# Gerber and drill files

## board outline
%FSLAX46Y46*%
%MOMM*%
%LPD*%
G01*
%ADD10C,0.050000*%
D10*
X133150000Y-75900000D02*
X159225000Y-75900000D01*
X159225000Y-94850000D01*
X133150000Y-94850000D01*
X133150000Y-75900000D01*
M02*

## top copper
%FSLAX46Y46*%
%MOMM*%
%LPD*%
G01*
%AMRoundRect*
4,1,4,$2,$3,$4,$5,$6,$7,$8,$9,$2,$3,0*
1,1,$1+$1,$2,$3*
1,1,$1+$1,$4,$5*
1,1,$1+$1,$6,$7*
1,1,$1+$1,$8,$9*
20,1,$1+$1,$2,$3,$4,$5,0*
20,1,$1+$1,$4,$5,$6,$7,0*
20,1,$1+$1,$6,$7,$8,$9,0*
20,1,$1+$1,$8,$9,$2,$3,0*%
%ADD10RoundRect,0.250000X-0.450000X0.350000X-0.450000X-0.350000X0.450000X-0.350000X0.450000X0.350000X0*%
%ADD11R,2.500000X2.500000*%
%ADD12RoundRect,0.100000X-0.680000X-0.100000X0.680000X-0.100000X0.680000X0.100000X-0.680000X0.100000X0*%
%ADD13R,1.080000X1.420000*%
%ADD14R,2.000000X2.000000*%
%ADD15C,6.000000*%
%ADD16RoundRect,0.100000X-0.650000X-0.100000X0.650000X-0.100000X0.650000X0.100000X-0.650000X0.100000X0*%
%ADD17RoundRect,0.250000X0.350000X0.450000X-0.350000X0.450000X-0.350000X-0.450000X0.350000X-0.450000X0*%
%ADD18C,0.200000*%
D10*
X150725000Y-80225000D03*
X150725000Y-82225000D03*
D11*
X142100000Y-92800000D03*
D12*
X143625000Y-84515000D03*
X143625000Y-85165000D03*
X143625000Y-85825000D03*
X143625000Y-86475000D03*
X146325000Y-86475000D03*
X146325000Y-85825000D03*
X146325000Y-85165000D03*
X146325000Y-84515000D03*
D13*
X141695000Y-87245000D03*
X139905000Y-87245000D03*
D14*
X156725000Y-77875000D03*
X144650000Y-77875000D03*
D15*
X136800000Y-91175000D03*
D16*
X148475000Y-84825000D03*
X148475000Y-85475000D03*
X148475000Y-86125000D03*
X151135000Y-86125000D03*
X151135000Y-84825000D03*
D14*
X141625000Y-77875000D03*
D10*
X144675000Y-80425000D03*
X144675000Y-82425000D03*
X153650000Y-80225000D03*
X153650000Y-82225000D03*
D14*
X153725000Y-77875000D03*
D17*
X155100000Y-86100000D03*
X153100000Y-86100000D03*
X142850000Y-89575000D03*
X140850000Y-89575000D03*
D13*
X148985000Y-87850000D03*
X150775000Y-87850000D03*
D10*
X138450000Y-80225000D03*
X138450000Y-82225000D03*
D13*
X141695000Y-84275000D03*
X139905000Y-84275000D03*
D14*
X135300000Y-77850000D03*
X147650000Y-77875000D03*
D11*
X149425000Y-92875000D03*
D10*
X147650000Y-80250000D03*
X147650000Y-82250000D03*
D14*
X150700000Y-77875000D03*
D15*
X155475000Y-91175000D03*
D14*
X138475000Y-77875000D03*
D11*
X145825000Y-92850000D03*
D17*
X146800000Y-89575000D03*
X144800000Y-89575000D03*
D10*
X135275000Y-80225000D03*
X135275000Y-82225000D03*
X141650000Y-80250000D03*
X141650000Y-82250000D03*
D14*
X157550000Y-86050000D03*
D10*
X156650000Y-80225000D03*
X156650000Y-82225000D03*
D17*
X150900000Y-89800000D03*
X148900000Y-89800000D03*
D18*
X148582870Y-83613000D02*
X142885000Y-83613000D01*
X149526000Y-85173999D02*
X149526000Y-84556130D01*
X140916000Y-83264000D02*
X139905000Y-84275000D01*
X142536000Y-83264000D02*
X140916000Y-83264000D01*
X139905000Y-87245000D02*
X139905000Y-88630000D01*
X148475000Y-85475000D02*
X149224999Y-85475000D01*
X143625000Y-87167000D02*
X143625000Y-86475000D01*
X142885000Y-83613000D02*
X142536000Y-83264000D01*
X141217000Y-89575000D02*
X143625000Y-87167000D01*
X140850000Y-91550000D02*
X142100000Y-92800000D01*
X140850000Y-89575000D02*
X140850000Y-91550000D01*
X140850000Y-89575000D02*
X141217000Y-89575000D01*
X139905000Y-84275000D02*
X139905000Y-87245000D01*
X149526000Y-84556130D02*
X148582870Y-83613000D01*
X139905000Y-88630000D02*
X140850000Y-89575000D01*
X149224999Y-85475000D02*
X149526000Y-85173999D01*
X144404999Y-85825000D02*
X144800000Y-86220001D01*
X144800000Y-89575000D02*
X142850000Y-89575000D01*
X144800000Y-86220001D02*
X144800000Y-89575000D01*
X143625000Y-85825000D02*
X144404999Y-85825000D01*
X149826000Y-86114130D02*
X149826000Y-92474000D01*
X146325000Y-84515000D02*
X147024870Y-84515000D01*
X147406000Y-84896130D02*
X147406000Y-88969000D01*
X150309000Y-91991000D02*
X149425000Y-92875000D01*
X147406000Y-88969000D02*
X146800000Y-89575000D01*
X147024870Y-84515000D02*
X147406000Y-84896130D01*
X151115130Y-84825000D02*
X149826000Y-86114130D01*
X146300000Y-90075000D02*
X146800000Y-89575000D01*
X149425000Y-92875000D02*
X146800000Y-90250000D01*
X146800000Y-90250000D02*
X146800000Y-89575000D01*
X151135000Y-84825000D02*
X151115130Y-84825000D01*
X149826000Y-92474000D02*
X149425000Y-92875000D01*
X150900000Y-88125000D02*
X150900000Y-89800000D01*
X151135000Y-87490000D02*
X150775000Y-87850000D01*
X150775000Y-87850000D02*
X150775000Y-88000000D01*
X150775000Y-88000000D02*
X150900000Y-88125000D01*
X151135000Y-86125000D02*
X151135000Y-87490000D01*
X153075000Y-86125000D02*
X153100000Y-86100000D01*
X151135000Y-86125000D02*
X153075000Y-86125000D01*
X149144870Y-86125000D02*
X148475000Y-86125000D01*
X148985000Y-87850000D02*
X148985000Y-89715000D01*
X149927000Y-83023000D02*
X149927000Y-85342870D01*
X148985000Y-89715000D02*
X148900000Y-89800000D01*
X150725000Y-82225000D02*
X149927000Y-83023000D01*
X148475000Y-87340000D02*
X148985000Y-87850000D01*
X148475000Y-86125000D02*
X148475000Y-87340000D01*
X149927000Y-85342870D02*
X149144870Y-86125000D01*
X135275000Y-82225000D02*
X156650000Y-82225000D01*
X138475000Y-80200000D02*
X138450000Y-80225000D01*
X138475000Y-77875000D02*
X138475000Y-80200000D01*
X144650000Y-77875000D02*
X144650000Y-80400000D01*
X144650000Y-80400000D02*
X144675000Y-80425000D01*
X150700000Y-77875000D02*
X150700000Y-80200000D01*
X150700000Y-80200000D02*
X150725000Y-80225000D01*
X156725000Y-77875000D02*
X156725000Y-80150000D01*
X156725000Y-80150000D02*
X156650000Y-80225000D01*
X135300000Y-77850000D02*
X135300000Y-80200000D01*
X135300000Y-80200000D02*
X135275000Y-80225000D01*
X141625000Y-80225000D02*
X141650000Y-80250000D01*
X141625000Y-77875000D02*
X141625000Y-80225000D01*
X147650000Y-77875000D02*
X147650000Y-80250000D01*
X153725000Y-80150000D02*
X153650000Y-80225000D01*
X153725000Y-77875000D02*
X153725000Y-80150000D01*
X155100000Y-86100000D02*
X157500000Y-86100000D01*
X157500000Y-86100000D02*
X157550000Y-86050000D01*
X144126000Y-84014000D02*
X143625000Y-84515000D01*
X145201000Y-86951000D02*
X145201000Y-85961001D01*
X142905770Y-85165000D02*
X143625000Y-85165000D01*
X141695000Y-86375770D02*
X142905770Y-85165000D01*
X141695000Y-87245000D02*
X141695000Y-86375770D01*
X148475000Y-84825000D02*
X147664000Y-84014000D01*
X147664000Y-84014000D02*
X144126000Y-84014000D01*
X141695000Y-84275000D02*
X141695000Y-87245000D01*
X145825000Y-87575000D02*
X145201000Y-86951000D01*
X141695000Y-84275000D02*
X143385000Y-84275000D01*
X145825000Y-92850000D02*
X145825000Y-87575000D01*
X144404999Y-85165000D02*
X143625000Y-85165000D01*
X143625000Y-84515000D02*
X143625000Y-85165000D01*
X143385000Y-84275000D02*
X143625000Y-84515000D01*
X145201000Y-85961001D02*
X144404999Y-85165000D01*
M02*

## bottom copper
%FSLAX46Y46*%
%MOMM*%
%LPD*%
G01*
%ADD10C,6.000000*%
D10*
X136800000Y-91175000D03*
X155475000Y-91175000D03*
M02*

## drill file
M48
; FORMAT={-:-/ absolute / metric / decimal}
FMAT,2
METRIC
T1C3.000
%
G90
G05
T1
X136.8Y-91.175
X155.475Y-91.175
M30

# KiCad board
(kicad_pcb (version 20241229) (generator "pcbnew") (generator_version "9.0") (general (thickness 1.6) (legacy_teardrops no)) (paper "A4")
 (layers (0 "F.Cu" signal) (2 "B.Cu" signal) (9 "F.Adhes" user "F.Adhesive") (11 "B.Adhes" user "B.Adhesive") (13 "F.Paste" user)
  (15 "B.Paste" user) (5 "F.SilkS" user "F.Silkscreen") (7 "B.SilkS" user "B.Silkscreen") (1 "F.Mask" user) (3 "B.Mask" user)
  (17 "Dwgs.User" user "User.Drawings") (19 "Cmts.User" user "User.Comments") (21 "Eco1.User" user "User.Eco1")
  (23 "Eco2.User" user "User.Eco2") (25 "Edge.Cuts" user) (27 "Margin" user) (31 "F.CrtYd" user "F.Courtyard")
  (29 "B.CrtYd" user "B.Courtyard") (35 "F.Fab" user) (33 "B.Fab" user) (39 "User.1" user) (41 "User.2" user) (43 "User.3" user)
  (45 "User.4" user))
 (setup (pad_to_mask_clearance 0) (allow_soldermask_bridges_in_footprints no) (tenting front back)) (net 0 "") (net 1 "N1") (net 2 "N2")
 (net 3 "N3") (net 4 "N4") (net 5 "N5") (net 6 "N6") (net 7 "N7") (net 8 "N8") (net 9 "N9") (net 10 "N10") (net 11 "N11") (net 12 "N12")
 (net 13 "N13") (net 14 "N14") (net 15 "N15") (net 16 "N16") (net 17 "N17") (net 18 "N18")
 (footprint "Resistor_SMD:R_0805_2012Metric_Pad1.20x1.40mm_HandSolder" (layer "F.Cu") (at 150.725 81.225 -90)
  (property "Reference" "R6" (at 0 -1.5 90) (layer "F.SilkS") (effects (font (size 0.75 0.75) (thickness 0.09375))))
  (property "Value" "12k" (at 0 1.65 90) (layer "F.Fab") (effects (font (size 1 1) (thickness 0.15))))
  (pad "1" smd roundrect (at -1 0 270) (size 1.2 1.4) (layers "F.Cu" "F.Mask" "F.Paste") (roundrect_rratio 0.208333) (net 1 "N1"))
  (pad "2" smd roundrect (at 1 0 270) (size 1.2 1.4) (layers "F.Cu" "F.Mask" "F.Paste") (roundrect_rratio 0.208333) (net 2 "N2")))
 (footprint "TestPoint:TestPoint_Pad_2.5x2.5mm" (layer "F.Cu") (at 142.1 92.8)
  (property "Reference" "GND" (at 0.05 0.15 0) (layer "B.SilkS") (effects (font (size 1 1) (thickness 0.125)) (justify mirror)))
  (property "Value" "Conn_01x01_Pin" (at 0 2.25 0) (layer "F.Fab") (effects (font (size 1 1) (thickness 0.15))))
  (pad "1" smd rect (at 0 0) (size 2.5 2.5) (layers "F.Cu" "F.Mask") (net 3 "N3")))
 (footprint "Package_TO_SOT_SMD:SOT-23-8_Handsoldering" (layer "F.Cu") (at 144.975 85.495)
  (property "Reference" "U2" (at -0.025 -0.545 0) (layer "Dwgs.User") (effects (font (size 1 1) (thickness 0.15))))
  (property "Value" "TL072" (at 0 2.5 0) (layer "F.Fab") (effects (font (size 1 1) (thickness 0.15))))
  (pad "1" smd roundrect (at -1.35 -0.98) (size 1.56 0.4) (layers "F.Cu" "F.Mask" "F.Paste") (roundrect_rratio 0.25) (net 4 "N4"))
  (pad "2" smd roundrect (at -1.35 -0.33) (size 1.56 0.4) (layers "F.Cu" "F.Mask" "F.Paste") (roundrect_rratio 0.25) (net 4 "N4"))
  (pad "3" smd roundrect (at -1.35 0.33) (size 1.56 0.4) (layers "F.Cu" "F.Mask" "F.Paste") (roundrect_rratio 0.25) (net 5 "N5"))
  (pad "4" smd roundrect (at -1.35 0.98) (size 1.56 0.4) (layers "F.Cu" "F.Mask" "F.Paste") (roundrect_rratio 0.25) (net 3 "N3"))
  (pad "5" smd roundrect (at 1.35 0.98) (size 1.56 0.4) (layers "F.Cu" "F.Mask" "F.Paste") (roundrect_rratio 0.25) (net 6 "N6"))
  (pad "6" smd roundrect (at 1.35 0.33) (size 1.56 0.4) (layers "F.Cu" "F.Mask" "F.Paste") (roundrect_rratio 0.25) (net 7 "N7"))
  (pad "7" smd roundrect (at 1.35 -0.33) (size 1.56 0.4) (layers "F.Cu" "F.Mask" "F.Paste") (roundrect_rratio 0.25) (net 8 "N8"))
  (pad "8" smd roundrect (at 1.35 -0.98) (size 1.56 0.4) (layers "F.Cu" "F.Mask" "F.Paste") (roundrect_rratio 0.25) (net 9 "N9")))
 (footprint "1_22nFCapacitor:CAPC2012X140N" (layer "F.Cu") (at 140.8 87.245 180)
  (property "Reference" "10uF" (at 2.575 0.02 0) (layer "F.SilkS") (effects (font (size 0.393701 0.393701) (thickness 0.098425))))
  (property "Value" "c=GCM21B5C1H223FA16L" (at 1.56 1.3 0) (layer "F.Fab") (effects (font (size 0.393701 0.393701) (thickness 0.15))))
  (pad "1" smd rect (at -0.895 0 180) (size 1.08 1.42) (layers "F.Cu" "F.Mask" "F.Paste") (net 4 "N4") (solder_mask_margin 0.102))
  (pad "2" smd rect (at 0.895 0 180) (size 1.08 1.42) (layers "F.Cu" "F.Mask" "F.Paste") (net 3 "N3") (solder_mask_margin 0.102)))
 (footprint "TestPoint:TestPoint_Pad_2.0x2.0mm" (layer "F.Cu") (at 156.725 77.875)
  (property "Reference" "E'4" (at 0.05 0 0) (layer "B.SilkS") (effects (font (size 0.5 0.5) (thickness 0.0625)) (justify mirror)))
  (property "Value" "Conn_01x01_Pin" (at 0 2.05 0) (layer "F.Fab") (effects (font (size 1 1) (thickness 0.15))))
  (pad "1" smd rect (at 0 0) (size 2 2) (layers "F.Cu" "F.Mask") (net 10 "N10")))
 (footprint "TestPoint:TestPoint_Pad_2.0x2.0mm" (layer "F.Cu") (at 144.65 77.875)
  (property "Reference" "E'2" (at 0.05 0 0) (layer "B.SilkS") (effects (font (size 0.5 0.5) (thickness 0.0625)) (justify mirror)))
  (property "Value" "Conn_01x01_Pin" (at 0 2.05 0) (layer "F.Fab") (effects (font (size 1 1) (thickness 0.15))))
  (pad "1" smd rect (at 0 0) (size 2 2) (layers "F.Cu" "F.Mask") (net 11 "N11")))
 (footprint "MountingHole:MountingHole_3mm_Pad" (layer "F.Cu") (at 136.8 91.175)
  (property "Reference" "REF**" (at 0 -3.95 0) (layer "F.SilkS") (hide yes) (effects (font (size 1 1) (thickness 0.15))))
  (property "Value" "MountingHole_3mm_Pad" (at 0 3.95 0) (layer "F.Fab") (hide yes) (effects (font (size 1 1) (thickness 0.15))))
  (pad "1" thru_hole circle (at 0 0) (size 6 6) (drill 3) (layers "*.Cu" "*.Mask") (remove_unused_layers no) (zone_connect 2)))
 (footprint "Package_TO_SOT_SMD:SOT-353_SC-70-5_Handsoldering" (layer "F.Cu") (at 149.805 85.475)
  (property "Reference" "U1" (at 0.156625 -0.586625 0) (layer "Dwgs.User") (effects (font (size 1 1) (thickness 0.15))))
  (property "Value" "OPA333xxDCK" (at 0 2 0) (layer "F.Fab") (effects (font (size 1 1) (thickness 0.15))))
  (pad "1" smd roundrect (at -1.33 -0.65) (size 1.5 0.4) (layers "F.Cu" "F.Mask" "F.Paste") (roundrect_rratio 0.25) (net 4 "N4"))
  (pad "2" smd roundrect (at -1.33 0) (size 1.5 0.4) (layers "F.Cu" "F.Mask" "F.Paste") (roundrect_rratio 0.25) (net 3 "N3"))
  (pad "3" smd roundrect (at -1.33 0.65) (size 1.5 0.4) (layers "F.Cu" "F.Mask" "F.Paste") (roundrect_rratio 0.25) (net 2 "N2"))
  (pad "4" smd roundrect (at 1.33 0.65) (size 1.5 0.4) (layers "F.Cu" "F.Mask" "F.Paste") (roundrect_rratio 0.25) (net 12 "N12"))
  (pad "5" smd roundrect (at 1.33 -0.65) (size 1.5 0.4) (layers "F.Cu" "F.Mask" "F.Paste") (roundrect_rratio 0.25) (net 9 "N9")))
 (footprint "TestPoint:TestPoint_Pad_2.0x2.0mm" (layer "F.Cu") (at 141.625 77.875)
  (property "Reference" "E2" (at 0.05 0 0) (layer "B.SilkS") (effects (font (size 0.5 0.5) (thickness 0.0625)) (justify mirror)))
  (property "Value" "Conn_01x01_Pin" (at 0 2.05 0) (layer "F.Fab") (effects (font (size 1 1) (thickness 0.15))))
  (pad "1" smd rect (at 0 0) (size 2 2) (layers "F.Cu" "F.Mask") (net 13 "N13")))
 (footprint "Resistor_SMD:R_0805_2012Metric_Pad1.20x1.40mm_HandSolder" (layer "F.Cu") (at 144.675 81.425 -90)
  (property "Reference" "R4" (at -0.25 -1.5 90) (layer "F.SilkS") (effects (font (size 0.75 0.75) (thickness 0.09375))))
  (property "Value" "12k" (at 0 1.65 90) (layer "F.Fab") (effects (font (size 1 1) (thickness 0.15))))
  (pad "1" smd roundrect (at -1 0 270) (size 1.2 1.4) (layers "F.Cu" "F.Mask" "F.Paste") (roundrect_rratio 0.208333) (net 11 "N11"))
  (pad "2" smd roundrect (at 1 0 270) (size 1.2 1.4) (layers "F.Cu" "F.Mask" "F.Paste") (roundrect_rratio 0.208333) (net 2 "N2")))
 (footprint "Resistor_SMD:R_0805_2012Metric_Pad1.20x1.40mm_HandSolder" (layer "F.Cu") (at 153.65 81.225 -90)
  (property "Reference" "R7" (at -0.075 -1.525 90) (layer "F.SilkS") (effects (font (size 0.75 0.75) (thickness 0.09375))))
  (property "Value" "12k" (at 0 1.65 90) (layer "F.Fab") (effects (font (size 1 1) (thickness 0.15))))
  (pad "1" smd roundrect (at -1 0 270) (size 1.2 1.4) (layers "F.Cu" "F.Mask" "F.Paste") (roundrect_rratio 0.208333) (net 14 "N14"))
  (pad "2" smd roundrect (at 1 0 270) (size 1.2 1.4) (layers "F.Cu" "F.Mask" "F.Paste") (roundrect_rratio 0.208333) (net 2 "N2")))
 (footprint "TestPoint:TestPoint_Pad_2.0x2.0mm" (layer "F.Cu") (at 153.725 77.875)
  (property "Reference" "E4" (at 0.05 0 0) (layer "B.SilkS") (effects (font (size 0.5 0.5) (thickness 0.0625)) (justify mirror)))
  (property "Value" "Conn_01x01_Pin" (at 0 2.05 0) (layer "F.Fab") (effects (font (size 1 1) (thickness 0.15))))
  (pad "1" smd rect (at 0 0) (size 2 2) (layers "F.Cu" "F.Mask") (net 14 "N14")))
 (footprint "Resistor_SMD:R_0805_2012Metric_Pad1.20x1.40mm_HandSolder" (layer "F.Cu") (at 154.1 86.1 180)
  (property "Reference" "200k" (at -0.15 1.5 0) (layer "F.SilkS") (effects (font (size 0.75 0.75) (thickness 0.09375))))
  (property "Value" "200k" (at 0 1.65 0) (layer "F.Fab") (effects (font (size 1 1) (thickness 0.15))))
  (pad "1" smd roundrect (at -1 0 180) (size 1.2 1.4) (layers "F.Cu" "F.Mask" "F.Paste") (roundrect_rratio 0.208333) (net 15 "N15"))
  (pad "2" smd roundrect (at 1 0 180) (size 1.2 1.4) (layers "F.Cu" "F.Mask" "F.Paste") (roundrect_rratio 0.208333) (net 12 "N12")))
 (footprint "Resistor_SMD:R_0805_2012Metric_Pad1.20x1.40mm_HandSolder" (layer "F.Cu") (at 141.85 89.575 180)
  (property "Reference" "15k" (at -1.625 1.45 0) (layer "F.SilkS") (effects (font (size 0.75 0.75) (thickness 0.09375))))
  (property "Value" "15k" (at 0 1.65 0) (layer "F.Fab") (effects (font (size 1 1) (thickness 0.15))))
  (pad "1" smd roundrect (at -1 0 180) (size 1.2 1.4) (layers "F.Cu" "F.Mask" "F.Paste") (roundrect_rratio 0.208333) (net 5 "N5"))
  (pad "2" smd roundrect (at 1 0 180) (size 1.2 1.4) (layers "F.Cu" "F.Mask" "F.Paste") (roundrect_rratio 0.208333) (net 3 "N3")))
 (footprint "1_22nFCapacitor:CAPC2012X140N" (layer "F.Cu") (at 149.88 87.85)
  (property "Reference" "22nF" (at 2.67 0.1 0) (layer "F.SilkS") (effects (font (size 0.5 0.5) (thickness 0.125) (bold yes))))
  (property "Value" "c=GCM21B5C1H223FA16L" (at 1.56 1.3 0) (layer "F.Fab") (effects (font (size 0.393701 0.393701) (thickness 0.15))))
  (pad "1" smd rect (at -0.895 0) (size 1.08 1.42) (layers "F.Cu" "F.Mask" "F.Paste") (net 2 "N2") (solder_mask_margin 0.102))
  (pad "2" smd rect (at 0.895 0) (size 1.08 1.42) (layers "F.Cu" "F.Mask" "F.Paste") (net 12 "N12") (solder_mask_margin 0.102)))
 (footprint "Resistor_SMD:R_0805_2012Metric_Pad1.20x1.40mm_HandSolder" (layer "F.Cu") (at 138.45 81.225 -90)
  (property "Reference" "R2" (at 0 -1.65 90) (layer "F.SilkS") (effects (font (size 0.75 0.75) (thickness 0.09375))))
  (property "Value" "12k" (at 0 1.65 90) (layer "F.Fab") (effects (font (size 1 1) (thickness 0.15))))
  (pad "1" smd roundrect (at -1 0 270) (size 1.2 1.4) (layers "F.Cu" "F.Mask" "F.Paste") (roundrect_rratio 0.208333) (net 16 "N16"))
  (pad "2" smd roundrect (at 1 0 270) (size 1.2 1.4) (layers "F.Cu" "F.Mask" "F.Paste") (roundrect_rratio 0.208333) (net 2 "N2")))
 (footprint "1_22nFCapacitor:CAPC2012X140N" (layer "F.Cu") (at 140.8 84.275 180)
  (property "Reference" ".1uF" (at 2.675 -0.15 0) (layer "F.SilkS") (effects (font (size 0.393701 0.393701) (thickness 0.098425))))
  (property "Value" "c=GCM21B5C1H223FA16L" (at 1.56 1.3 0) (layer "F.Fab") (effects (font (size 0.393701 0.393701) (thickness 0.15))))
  (pad "1" smd rect (at -0.895 0 180) (size 1.08 1.42) (layers "F.Cu" "F.Mask" "F.Paste") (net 4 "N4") (solder_mask_margin 0.102))
  (pad "2" smd rect (at 0.895 0 180) (size 1.08 1.42) (layers "F.Cu" "F.Mask" "F.Paste") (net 3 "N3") (solder_mask_margin 0.102)))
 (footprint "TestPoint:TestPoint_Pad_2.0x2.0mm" (layer "F.Cu") (at 135.3 77.85)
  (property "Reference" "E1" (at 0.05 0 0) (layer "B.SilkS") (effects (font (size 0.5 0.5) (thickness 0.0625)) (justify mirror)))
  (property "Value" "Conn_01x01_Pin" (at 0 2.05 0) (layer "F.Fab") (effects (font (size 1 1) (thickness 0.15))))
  (pad "1" smd rect (at 0 0) (size 2 2) (layers "F.Cu" "F.Mask") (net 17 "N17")))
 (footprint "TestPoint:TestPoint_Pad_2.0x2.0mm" (layer "F.Cu") (at 147.65 77.875)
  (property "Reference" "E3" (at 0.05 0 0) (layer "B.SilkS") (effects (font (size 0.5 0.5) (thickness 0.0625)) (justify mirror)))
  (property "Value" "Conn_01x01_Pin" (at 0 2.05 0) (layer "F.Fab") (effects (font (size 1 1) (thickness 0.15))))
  (pad "1" smd rect (at 0 0) (size 2 2) (layers "F.Cu" "F.Mask") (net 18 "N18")))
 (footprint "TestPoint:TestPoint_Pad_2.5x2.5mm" (layer "F.Cu") (at 149.425 92.875)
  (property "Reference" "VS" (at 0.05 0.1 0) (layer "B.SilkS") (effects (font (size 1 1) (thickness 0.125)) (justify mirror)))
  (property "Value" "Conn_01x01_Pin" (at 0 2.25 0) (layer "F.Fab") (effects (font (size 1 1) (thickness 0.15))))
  (pad "1" smd rect (at 0 0) (size 2.5 2.5) (layers "F.Cu" "F.Mask") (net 9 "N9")))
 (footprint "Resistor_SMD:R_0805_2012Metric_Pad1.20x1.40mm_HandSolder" (layer "F.Cu") (at 147.65 81.25 -90)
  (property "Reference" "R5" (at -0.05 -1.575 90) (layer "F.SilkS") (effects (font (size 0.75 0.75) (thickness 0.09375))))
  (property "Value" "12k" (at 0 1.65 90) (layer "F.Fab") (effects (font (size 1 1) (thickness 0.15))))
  (pad "1" smd roundrect (at -1 0 270) (size 1.2 1.4) (layers "F.Cu" "F.Mask" "F.Paste") (roundrect_rratio 0.208333) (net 18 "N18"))
  (pad "2" smd roundrect (at 1 0 270) (size 1.2 1.4) (layers "F.Cu" "F.Mask" "F.Paste") (roundrect_rratio 0.208333) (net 2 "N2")))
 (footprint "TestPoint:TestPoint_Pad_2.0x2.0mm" (layer "F.Cu") (at 150.7 77.875)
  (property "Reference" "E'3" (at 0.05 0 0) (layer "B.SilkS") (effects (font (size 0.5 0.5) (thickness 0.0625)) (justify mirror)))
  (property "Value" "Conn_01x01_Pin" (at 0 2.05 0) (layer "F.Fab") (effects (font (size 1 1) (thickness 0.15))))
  (pad "1" smd rect (at 0 0) (size 2 2) (layers "F.Cu" "F.Mask") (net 1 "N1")))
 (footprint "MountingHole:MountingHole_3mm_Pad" (layer "F.Cu") (at 155.475 91.175)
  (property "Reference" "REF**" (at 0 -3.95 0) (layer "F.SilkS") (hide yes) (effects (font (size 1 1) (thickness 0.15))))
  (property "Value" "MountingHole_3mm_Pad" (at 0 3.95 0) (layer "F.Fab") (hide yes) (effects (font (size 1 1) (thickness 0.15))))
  (pad "1" thru_hole circle (at 0 0) (size 6 6) (drill 3) (layers "*.Cu" "*.Mask") (remove_unused_layers no) (zone_connect 2)))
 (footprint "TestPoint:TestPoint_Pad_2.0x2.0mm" (layer "F.Cu") (at 138.475 77.875)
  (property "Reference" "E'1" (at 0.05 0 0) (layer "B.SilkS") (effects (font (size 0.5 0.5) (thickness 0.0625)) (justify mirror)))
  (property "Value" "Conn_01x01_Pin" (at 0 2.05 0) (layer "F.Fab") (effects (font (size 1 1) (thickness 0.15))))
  (pad "1" smd rect (at 0 0) (size 2 2) (layers "F.Cu" "F.Mask") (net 16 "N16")))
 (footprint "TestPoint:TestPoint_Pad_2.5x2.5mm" (layer "F.Cu") (at 145.825 92.85)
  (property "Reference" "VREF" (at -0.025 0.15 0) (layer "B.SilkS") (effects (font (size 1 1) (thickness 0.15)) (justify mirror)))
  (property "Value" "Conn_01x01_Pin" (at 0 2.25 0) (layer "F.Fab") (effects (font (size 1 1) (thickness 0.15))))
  (pad "1" smd rect (at 0 0) (size 2.5 2.5) (layers "F.Cu" "F.Mask") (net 4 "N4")))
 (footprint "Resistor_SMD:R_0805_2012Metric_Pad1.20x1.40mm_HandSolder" (layer "F.Cu") (at 145.8 89.575 180)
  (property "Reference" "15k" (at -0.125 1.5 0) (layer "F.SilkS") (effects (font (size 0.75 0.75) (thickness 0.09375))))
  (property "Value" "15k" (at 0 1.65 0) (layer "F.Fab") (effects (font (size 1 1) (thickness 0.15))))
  (pad "1" smd roundrect (at -1 0 180) (size 1.2 1.4) (layers "F.Cu" "F.Mask" "F.Paste") (roundrect_rratio 0.208333) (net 9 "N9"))
  (pad "2" smd roundrect (at 1 0 180) (size 1.2 1.4) (layers "F.Cu" "F.Mask" "F.Paste") (roundrect_rratio 0.208333) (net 5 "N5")))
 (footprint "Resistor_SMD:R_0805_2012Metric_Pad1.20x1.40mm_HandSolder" (layer "F.Cu") (at 135.275 81.225 -90)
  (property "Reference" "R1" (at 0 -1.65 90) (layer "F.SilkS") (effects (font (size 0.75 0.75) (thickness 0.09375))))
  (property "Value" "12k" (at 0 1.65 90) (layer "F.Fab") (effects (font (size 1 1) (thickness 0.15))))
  (pad "1" smd roundrect (at -1 0 270) (size 1.2 1.4) (layers "F.Cu" "F.Mask" "F.Paste") (roundrect_rratio 0.208333) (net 17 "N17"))
  (pad "2" smd roundrect (at 1 0 270) (size 1.2 1.4) (layers "F.Cu" "F.Mask" "F.Paste") (roundrect_rratio 0.208333) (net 2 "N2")))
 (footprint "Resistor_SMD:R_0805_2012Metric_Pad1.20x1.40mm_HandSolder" (layer "F.Cu") (at 141.65 81.25 -90)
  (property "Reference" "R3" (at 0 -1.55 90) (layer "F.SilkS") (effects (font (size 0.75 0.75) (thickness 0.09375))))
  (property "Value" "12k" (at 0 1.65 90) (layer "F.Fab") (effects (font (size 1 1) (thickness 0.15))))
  (pad "1" smd roundrect (at -1 0 270) (size 1.2 1.4) (layers "F.Cu" "F.Mask" "F.Paste") (roundrect_rratio 0.208333) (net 13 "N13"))
  (pad "2" smd roundrect (at 1 0 270) (size 1.2 1.4) (layers "F.Cu" "F.Mask" "F.Paste") (roundrect_rratio 0.208333) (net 2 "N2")))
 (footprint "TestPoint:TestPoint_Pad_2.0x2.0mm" (layer "F.Cu") (at 157.55 86.05)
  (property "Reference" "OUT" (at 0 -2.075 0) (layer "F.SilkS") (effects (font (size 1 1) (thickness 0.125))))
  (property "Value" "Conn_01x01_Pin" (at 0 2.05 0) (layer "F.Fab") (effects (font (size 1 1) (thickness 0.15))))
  (pad "1" smd rect (at 0 0) (size 2 2) (layers "F.Cu" "F.Mask") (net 15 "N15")))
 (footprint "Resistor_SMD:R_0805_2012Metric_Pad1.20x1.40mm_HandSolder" (layer "F.Cu") (at 156.65 81.225 -90)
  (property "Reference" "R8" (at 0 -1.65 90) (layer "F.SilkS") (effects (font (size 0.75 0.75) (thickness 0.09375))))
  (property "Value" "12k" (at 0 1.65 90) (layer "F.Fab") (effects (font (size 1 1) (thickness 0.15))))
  (pad "1" smd roundrect (at -1 0 270) (size 1.2 1.4) (layers "F.Cu" "F.Mask" "F.Paste") (roundrect_rratio 0.208333) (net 10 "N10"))
  (pad "2" smd roundrect (at 1 0 270) (size 1.2 1.4) (layers "F.Cu" "F.Mask" "F.Paste") (roundrect_rratio 0.208333) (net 2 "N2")))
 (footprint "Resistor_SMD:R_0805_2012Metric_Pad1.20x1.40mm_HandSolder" (layer "F.Cu") (at 149.9 89.8 180)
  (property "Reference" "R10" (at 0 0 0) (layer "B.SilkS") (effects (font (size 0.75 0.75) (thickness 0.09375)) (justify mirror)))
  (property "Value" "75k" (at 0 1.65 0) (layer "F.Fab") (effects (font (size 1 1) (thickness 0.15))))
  (pad "1" smd roundrect (at -1 0 180) (size 1.2 1.4) (layers "F.Cu" "F.Mask" "F.Paste") (roundrect_rratio 0.208333) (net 12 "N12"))
  (pad "2" smd roundrect (at 1 0 180) (size 1.2 1.4) (layers "F.Cu" "F.Mask" "F.Paste") (roundrect_rratio 0.208333) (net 2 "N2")))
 (gr_rect (start 133.15 75.9) (end 159.225 94.85) (stroke (width 0.05) (type solid)) (fill no) (layer "Edge.Cuts"))
 (segment (start 148.58287 83.613) (end 142.885 83.613) (width 0.2) (layer "F.Cu") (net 3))
 (segment (start 149.526 85.173999) (end 149.526 84.55613) (width 0.2) (layer "F.Cu") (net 3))
 (segment (start 140.916 83.264) (end 139.905 84.275) (width 0.2) (layer "F.Cu") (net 3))
 (segment (start 142.536 83.264) (end 140.916 83.264) (width 0.2) (layer "F.Cu") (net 3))
 (segment (start 139.905 87.245) (end 139.905 88.63) (width 0.2) (layer "F.Cu") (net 3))
 (segment (start 148.475 85.475) (end 149.224999 85.475) (width 0.2) (layer "F.Cu") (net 3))
 (segment (start 143.625 87.167) (end 143.625 86.475) (width 0.2) (layer "F.Cu") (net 3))
 (segment (start 142.885 83.613) (end 142.536 83.264) (width 0.2) (layer "F.Cu") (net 3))
 (segment (start 141.217 89.575) (end 143.625 87.167) (width 0.2) (layer "F.Cu") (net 3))
 (segment (start 140.85 91.55) (end 142.1 92.8) (width 0.2) (layer "F.Cu") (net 3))
 (segment (start 140.85 89.575) (end 140.85 91.55) (width 0.2) (layer "F.Cu") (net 3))
 (segment (start 140.85 89.575) (end 141.217 89.575) (width 0.2) (layer "F.Cu") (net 3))
 (segment (start 139.905 84.275) (end 139.905 87.245) (width 0.2) (layer "F.Cu") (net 3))
 (segment (start 149.526 84.55613) (end 148.58287 83.613) (width 0.2) (layer "F.Cu") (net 3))
 (segment (start 139.905 88.63) (end 140.85 89.575) (width 0.2) (layer "F.Cu") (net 3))
 (segment (start 149.224999 85.475) (end 149.526 85.173999) (width 0.2) (layer "F.Cu") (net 3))
 (segment (start 144.404999 85.825) (end 144.8 86.220001) (width 0.2) (layer "F.Cu") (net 5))
 (segment (start 144.8 89.575) (end 142.85 89.575) (width 0.2) (layer "F.Cu") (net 5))
 (segment (start 144.8 86.220001) (end 144.8 89.575) (width 0.2) (layer "F.Cu") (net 5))
 (segment (start 143.625 85.825) (end 144.404999 85.825) (width 0.2) (layer "F.Cu") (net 5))
 (segment (start 149.826 86.11413) (end 149.826 92.474) (width 0.2) (layer "F.Cu") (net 9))
 (segment (start 146.325 84.515) (end 147.02487 84.515) (width 0.2) (layer "F.Cu") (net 9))
 (segment (start 147.406 84.89613) (end 147.406 88.969) (width 0.2) (layer "F.Cu") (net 9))
 (segment (start 150.309 91.991) (end 149.425 92.875) (width 0.2) (layer "F.Cu") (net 9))
 (segment (start 147.406 88.969) (end 146.8 89.575) (width 0.2) (layer "F.Cu") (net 9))
 (segment (start 147.02487 84.515) (end 147.406 84.89613) (width 0.2) (layer "F.Cu") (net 9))
 (segment (start 151.11513 84.825) (end 149.826 86.11413) (width 0.2) (layer "F.Cu") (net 9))
 (segment (start 146.3 90.075) (end 146.8 89.575) (width 0.2) (layer "F.Cu") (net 9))
 (segment (start 149.425 92.875) (end 146.8 90.25) (width 0.2) (layer "F.Cu") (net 9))
 (segment (start 146.8 90.25) (end 146.8 89.575) (width 0.2) (layer "F.Cu") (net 9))
 (segment (start 151.135 84.825) (end 151.11513 84.825) (width 0.2) (layer "F.Cu") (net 9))
 (segment (start 149.826 92.474) (end 149.425 92.875) (width 0.2) (layer "F.Cu") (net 9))
 (segment (start 150.9 88.125) (end 150.9 89.8) (width 0.2) (layer "F.Cu") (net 12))
 (segment (start 151.135 87.49) (end 150.775 87.85) (width 0.2) (layer "F.Cu") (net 12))
 (segment (start 150.775 87.85) (end 150.775 88) (width 0.2) (layer "F.Cu") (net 12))
 (segment (start 150.775 88) (end 150.9 88.125) (width 0.2) (layer "F.Cu") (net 12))
 (segment (start 151.135 86.125) (end 151.135 87.49) (width 0.2) (layer "F.Cu") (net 12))
 (segment (start 153.075 86.125) (end 153.1 86.1) (width 0.2) (layer "F.Cu") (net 12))
 (segment (start 151.135 86.125) (end 153.075 86.125) (width 0.2) (layer "F.Cu") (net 12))
 (segment (start 149.14487 86.125) (end 148.475 86.125) (width 0.2) (layer "F.Cu") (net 2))
 (segment (start 148.985 87.85) (end 148.985 89.715) (width 0.2) (layer "F.Cu") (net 2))
 (segment (start 149.927 83.023) (end 149.927 85.34287) (width 0.2) (layer "F.Cu") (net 2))
 (segment (start 148.985 89.715) (end 148.9 89.8) (width 0.2) (layer "F.Cu") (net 2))
 (segment (start 150.725 82.225) (end 149.927 83.023) (width 0.2) (layer "F.Cu") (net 2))
 (segment (start 148.475 87.34) (end 148.985 87.85) (width 0.2) (layer "F.Cu") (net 2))
 (segment (start 148.475 86.125) (end 148.475 87.34) (width 0.2) (layer "F.Cu") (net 2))
 (segment (start 149.927 85.34287) (end 149.14487 86.125) (width 0.2) (layer "F.Cu") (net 2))
 (segment (start 135.275 82.225) (end 156.65 82.225) (width 0.2) (layer "F.Cu") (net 2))
 (segment (start 138.475 80.2) (end 138.45 80.225) (width 0.2) (layer "F.Cu") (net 16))
 (segment (start 138.475 77.875) (end 138.475 80.2) (width 0.2) (layer "F.Cu") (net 16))
 (segment (start 144.65 77.875) (end 144.65 80.4) (width 0.2) (layer "F.Cu") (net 11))
 (segment (start 144.65 80.4) (end 144.675 80.425) (width 0.2) (layer "F.Cu") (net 11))
 (segment (start 150.7 77.875) (end 150.7 80.2) (width 0.2) (layer "F.Cu") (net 1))
 (segment (start 150.7 80.2) (end 150.725 80.225) (width 0.2) (layer "F.Cu") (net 1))
 (segment (start 156.725 77.875) (end 156.725 80.15) (width 0.2) (layer "F.Cu") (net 10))
 (segment (start 156.725 80.15) (end 156.65 80.225) (width 0.2) (layer "F.Cu") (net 10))
 (segment (start 135.3 77.85) (end 135.3 80.2) (width 0.2) (layer "F.Cu") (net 17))
 (segment (start 135.3 80.2) (end 135.275 80.225) (width 0.2) (layer "F.Cu") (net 17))
 (segment (start 141.625 80.225) (end 141.65 80.25) (width 0.2) (layer "F.Cu") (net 13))
 (segment (start 141.625 77.875) (end 141.625 80.225) (width 0.2) (layer "F.Cu") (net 13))
 (segment (start 147.65 77.875) (end 147.65 80.25) (width 0.2) (layer "F.Cu") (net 18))
 (segment (start 153.725 80.15) (end 153.65 80.225) (width 0.2) (layer "F.Cu") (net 14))
 (segment (start 153.725 77.875) (end 153.725 80.15) (width 0.2) (layer "F.Cu") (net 14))
 (segment (start 155.1 86.1) (end 157.5 86.1) (width 0.2) (layer "F.Cu") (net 15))
 (segment (start 157.5 86.1) (end 157.55 86.05) (width 0.2) (layer "F.Cu") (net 15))
 (segment (start 144.126 84.014) (end 143.625 84.515) (width 0.2) (layer "F.Cu") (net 4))
 (segment (start 145.201 86.951) (end 145.201 85.961001) (width 0.2) (layer "F.Cu") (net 4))
 (segment (start 142.90577 85.165) (end 143.625 85.165) (width 0.2) (layer "F.Cu") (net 4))
 (segment (start 141.695 86.37577) (end 142.90577 85.165) (width 0.2) (layer "F.Cu") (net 4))
 (segment (start 141.695 87.245) (end 141.695 86.37577) (width 0.2) (layer "F.Cu") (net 4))
 (segment (start 148.475 84.825) (end 147.664 84.014) (width 0.2) (layer "F.Cu") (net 4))
 (segment (start 147.664 84.014) (end 144.126 84.014) (width 0.2) (layer "F.Cu") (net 4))
 (segment (start 141.695 84.275) (end 141.695 87.245) (width 0.2) (layer "F.Cu") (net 4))
 (segment (start 145.825 87.575) (end 145.201 86.951) (width 0.2) (layer "F.Cu") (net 4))
 (segment (start 141.695 84.275) (end 143.385 84.275) (width 0.2) (layer "F.Cu") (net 4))
 (segment (start 145.825 92.85) (end 145.825 87.575) (width 0.2) (layer "F.Cu") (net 4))
 (segment (start 144.404999 85.165) (end 143.625 85.165) (width 0.2) (layer "F.Cu") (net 4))
 (segment (start 143.625 84.515) (end 143.625 85.165) (width 0.2) (layer "F.Cu") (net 4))
 (segment (start 143.385 84.275) (end 143.625 84.515) (width 0.2) (layer "F.Cu") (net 4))
 (segment (start 145.201 85.961001) (end 144.404999 85.165) (width 0.2) (layer "F.Cu") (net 4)))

